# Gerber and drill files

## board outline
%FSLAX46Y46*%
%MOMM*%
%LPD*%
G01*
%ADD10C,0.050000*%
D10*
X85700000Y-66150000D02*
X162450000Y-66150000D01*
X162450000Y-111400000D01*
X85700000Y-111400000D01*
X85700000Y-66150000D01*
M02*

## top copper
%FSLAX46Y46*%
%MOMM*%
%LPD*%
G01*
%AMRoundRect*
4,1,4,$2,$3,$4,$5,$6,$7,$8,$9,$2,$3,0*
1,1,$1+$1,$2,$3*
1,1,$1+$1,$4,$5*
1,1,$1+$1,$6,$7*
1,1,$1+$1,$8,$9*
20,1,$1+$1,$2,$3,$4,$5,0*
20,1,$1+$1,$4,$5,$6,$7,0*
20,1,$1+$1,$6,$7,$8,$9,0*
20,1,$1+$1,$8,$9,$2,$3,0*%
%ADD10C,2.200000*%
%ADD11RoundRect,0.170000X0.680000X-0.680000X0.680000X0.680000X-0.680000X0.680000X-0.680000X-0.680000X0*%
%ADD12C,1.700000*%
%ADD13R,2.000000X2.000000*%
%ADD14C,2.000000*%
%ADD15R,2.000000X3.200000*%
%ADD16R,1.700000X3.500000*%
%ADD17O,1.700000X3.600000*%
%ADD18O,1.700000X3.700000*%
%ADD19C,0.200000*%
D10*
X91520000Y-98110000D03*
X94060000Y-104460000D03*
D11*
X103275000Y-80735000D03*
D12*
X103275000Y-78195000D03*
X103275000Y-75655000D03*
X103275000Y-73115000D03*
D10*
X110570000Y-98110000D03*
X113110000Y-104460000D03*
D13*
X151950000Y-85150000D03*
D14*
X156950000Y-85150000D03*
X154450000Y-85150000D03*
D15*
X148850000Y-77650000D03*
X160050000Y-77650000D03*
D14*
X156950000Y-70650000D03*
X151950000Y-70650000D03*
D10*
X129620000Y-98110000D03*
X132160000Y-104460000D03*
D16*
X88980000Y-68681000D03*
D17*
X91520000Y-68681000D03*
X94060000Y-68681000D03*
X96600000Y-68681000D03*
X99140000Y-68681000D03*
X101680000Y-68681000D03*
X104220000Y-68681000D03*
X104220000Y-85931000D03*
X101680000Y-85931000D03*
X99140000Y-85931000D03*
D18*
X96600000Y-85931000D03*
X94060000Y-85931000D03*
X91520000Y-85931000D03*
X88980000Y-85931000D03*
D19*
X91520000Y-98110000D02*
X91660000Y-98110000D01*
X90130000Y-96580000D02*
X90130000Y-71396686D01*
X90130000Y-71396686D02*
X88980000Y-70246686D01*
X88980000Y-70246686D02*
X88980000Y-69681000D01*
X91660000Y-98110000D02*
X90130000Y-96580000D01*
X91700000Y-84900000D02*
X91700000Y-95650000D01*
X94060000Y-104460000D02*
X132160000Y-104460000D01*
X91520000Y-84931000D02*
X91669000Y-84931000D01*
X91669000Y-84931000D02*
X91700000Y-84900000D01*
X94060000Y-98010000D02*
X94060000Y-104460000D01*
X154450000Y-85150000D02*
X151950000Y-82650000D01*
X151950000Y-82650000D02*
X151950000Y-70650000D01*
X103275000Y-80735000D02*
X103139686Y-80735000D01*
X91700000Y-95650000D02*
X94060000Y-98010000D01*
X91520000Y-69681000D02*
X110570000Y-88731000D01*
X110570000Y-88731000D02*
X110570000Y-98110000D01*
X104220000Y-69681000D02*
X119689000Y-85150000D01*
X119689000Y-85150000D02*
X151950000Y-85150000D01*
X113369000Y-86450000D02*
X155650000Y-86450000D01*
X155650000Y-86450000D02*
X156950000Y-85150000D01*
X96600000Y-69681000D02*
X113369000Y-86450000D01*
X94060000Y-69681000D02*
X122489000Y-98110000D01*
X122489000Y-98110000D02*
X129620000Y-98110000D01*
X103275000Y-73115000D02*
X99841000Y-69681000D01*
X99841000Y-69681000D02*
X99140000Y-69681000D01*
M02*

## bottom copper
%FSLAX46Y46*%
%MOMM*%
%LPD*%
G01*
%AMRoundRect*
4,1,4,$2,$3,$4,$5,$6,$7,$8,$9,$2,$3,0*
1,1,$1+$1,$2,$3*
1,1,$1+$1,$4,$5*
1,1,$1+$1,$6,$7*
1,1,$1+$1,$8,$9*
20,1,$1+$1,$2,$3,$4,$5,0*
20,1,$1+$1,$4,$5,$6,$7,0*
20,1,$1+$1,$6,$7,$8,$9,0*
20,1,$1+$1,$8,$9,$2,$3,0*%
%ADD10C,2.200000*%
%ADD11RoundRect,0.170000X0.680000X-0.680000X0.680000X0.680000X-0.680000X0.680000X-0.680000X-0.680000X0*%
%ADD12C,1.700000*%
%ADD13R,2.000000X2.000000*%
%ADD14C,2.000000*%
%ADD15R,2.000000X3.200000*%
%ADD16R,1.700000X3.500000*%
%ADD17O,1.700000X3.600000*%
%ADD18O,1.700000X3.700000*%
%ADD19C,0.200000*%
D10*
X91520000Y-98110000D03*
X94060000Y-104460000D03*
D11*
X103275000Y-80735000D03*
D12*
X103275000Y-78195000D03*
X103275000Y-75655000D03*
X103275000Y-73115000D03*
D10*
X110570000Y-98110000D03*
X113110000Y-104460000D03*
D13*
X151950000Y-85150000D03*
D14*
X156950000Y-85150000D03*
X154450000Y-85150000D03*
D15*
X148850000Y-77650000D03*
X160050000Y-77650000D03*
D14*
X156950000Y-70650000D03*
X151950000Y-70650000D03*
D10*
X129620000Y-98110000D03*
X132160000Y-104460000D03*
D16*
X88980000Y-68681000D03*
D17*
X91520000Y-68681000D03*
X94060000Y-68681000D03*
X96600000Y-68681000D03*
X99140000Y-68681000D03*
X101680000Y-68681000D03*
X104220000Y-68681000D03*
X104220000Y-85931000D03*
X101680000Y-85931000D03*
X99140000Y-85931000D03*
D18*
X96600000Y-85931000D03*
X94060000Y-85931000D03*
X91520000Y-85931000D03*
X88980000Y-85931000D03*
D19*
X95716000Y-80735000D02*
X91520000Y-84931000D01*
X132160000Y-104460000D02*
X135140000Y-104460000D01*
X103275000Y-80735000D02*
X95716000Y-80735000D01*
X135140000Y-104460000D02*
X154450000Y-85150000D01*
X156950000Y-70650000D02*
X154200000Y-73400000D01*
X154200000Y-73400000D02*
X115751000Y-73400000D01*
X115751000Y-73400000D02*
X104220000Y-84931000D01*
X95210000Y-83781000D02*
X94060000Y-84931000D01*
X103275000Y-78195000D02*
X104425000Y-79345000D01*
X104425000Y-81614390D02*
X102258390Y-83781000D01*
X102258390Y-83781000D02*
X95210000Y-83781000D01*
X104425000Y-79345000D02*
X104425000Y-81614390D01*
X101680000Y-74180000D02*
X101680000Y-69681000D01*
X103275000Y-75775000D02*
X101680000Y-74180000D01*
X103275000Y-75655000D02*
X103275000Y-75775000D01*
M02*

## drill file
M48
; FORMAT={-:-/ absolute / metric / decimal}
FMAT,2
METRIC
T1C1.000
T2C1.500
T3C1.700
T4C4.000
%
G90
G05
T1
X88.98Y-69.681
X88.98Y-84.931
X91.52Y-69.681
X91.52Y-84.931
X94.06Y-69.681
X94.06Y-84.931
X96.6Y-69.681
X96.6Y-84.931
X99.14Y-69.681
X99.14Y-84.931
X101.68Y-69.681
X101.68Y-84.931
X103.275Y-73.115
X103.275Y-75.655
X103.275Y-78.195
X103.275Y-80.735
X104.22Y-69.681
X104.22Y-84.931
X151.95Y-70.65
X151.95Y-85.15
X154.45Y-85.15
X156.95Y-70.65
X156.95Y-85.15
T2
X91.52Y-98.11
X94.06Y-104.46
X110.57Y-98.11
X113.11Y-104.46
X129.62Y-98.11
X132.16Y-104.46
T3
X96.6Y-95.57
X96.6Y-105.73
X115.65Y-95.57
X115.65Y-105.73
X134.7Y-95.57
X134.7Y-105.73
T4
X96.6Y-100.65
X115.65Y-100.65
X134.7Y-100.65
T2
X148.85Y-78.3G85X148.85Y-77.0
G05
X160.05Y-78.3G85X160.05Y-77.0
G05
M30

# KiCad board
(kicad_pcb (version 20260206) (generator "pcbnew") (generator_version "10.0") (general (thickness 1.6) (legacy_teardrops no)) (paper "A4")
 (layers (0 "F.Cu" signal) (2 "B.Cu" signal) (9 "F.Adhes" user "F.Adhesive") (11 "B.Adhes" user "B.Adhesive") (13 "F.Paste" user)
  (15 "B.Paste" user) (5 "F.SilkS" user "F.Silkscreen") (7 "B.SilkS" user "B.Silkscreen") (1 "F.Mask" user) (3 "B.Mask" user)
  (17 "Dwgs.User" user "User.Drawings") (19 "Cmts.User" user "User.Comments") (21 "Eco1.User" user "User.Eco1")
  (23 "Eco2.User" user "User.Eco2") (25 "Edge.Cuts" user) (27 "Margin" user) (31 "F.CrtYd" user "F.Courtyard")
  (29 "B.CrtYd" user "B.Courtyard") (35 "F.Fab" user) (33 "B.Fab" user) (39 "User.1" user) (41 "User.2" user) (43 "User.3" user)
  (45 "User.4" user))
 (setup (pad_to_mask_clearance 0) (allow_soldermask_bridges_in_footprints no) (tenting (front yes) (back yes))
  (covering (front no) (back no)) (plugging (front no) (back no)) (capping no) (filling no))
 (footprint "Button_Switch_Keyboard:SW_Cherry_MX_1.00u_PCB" (layer "F.Cu") (at 91.52 98.11 90)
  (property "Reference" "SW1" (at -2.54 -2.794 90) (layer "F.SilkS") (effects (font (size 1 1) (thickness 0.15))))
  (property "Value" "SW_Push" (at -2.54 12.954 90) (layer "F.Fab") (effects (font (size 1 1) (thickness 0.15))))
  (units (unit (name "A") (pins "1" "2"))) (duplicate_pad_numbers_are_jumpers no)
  (pad "" np_thru_hole circle (at -7.62 5.08 90) (size 1.7 1.7) (drill 1.7) (layers "*.Cu" "*.Mask"))
  (pad "" np_thru_hole circle (at -2.54 5.08 90) (size 4 4) (drill 4) (layers "*.Cu" "*.Mask"))
  (pad "" np_thru_hole circle (at 2.54 5.08 90) (size 1.7 1.7) (drill 1.7) (layers "*.Cu" "*.Mask"))
  (pad "1" thru_hole circle (at 0 0 90) (size 2.2 2.2) (drill 1.5) (layers "*.Cu" "*.Mask") (remove_unused_layers no)
   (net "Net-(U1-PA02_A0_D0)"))
  (pad "2" thru_hole circle (at -6.35 2.54 90) (size 2.2 2.2) (drill 1.5) (layers "*.Cu" "*.Mask") (remove_unused_layers no) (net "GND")))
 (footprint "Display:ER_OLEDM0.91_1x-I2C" (layer "F.Cu") (at 103.275 80.735 90)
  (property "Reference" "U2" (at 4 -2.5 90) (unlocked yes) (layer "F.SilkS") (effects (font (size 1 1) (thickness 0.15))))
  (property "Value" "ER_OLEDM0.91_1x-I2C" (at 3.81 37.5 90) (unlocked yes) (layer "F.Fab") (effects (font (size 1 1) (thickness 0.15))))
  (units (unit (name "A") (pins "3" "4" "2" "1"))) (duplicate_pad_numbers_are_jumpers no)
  (pad "1" thru_hole roundrect (at 0 0 90) (size 1.7 1.7) (drill 1) (layers "*.Cu" "*.Mask") (remove_unused_layers no)
   (roundrect_rratio 0.1) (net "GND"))
  (pad "2" thru_hole circle (at 2.54 0 90) (size 1.7 1.7) (drill 1) (layers "*.Cu" "*.Mask") (remove_unused_layers no) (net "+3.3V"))
  (pad "3" thru_hole circle (at 5.08 0 90) (size 1.7 1.7) (drill 1) (layers "*.Cu" "*.Mask") (remove_unused_layers no)
   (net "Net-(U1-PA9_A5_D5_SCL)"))
  (pad "4" thru_hole circle (at 7.62 0 90) (size 1.7 1.7) (drill 1) (layers "*.Cu" "*.Mask") (remove_unused_layers no)
   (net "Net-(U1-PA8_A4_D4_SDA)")))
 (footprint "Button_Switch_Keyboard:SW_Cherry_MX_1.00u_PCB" (layer "F.Cu") (at 110.57 98.11 90)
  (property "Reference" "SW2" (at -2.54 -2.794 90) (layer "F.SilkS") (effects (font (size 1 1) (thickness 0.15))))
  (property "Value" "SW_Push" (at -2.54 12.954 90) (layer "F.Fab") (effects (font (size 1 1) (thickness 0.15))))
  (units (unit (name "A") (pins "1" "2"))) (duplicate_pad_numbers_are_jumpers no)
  (pad "" np_thru_hole circle (at -7.62 5.08 90) (size 1.7 1.7) (drill 1.7) (layers "*.Cu" "*.Mask"))
  (pad "" np_thru_hole circle (at -2.54 5.08 90) (size 4 4) (drill 4) (layers "*.Cu" "*.Mask"))
  (pad "" np_thru_hole circle (at 2.54 5.08 90) (size 1.7 1.7) (drill 1.7) (layers "*.Cu" "*.Mask"))
  (pad "1" thru_hole circle (at 0 0 90) (size 2.2 2.2) (drill 1.5) (layers "*.Cu" "*.Mask") (remove_unused_layers no)
   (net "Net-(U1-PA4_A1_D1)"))
  (pad "2" thru_hole circle (at -6.35 2.54 90) (size 2.2 2.2) (drill 1.5) (layers "*.Cu" "*.Mask") (remove_unused_layers no) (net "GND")))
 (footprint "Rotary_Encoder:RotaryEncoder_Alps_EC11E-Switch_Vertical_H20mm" (layer "F.Cu") (at 151.95 85.15 90)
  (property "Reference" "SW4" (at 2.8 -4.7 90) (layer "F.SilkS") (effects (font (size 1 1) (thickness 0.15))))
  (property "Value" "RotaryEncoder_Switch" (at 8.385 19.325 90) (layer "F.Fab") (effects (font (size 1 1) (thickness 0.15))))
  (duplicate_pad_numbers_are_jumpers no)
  (pad "A" thru_hole rect (at 0 0 90) (size 2 2) (drill 1) (layers "*.Cu" "*.Mask") (remove_unused_layers no) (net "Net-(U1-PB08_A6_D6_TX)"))
  (pad "B" thru_hole circle (at 0 5 90) (size 2 2) (drill 1) (layers "*.Cu" "*.Mask") (remove_unused_layers no) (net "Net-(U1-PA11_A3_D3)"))
  (pad "C" thru_hole circle (at 0 2.5 90) (size 2 2) (drill 1) (layers "*.Cu" "*.Mask") (remove_unused_layers no) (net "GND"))
  (pad "MP" thru_hole rect (at 7.5 -3.1 90) (size 3.2 2) (drill oval 2.8 1.5) (layers "*.Cu" "*.Mask") (remove_unused_layers no))
  (pad "MP" thru_hole rect (at 7.5 8.1 90) (size 3.2 2) (drill oval 2.8 1.5) (layers "*.Cu" "*.Mask") (remove_unused_layers no))
  (pad "S1" thru_hole circle (at 14.5 5 90) (size 2 2) (drill 1) (layers "*.Cu" "*.Mask") (remove_unused_layers no)
   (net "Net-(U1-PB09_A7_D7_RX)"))
  (pad "S2" thru_hole circle (at 14.5 0 90) (size 2 2) (drill 1) (layers "*.Cu" "*.Mask") (remove_unused_layers no) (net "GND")))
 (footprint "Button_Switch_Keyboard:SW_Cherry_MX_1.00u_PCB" (layer "F.Cu") (at 129.62 98.11 90)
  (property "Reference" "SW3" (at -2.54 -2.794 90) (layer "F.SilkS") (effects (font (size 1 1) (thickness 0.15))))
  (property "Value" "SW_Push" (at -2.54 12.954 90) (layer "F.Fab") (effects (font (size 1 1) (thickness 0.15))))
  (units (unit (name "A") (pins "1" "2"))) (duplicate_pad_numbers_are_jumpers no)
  (pad "" np_thru_hole circle (at -7.62 5.08 90) (size 1.7 1.7) (drill 1.7) (layers "*.Cu" "*.Mask"))
  (pad "" np_thru_hole circle (at -2.54 5.08 90) (size 4 4) (drill 4) (layers "*.Cu" "*.Mask"))
  (pad "" np_thru_hole circle (at 2.54 5.08 90) (size 1.7 1.7) (drill 1.7) (layers "*.Cu" "*.Mask"))
  (pad "1" thru_hole circle (at 0 0 90) (size 2.2 2.2) (drill 1.5) (layers "*.Cu" "*.Mask") (remove_unused_layers no)
   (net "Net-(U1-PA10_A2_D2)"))
  (pad "2" thru_hole circle (at -6.35 2.54 90) (size 2.2 2.2) (drill 1.5) (layers "*.Cu" "*.Mask") (remove_unused_layers no) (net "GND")))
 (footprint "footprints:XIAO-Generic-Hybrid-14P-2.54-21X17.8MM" (layer "B.Cu") (at 96.6 77.306 -90)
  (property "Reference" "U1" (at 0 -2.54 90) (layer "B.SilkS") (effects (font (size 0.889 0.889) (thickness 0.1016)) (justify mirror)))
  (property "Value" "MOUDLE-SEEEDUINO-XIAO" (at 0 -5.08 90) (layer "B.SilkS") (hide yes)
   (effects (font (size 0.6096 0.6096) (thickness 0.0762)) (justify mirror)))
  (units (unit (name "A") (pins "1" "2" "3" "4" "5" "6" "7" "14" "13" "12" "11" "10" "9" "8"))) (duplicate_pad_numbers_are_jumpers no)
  (pad "1" thru_hole rect (at -7.625 7.62 270) (size 3.5 1.7) (drill 1 (offset -1 0)) (layers "*.Cu" "*.Mask") (remove_unused_layers no)
   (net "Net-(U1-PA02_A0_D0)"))
  (pad "2" thru_hole oval (at -7.625 5.08 270) (size 3.6 1.7) (drill 1 (offset -1 0)) (layers "*.Cu" "*.Mask") (remove_unused_layers no)
   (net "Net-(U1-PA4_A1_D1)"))
  (pad "3" thru_hole oval (at -7.625 2.54 270) (size 3.6 1.7) (drill 1 (offset -1 0)) (layers "*.Cu" "*.Mask") (remove_unused_layers no)
   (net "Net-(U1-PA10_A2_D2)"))
  (pad "4" thru_hole oval (at -7.625 0 270) (size 3.6 1.7) (drill 1 (offset -1 0)) (layers "*.Cu" "*.Mask") (remove_unused_layers no)
   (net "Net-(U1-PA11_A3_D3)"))
  (pad "5" thru_hole oval (at -7.625 -2.54 270) (size 3.6 1.7) (drill 1 (offset -1 0)) (layers "*.Cu" "*.Mask") (remove_unused_layers no)
   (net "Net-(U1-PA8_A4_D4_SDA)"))
  (pad "6" thru_hole oval (at -7.625 -5.08 90) (size 3.6 1.7) (drill 1 (offset 1 0)) (layers "*.Cu" "*.Mask") (remove_unused_layers no)
   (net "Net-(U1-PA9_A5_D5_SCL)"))
  (pad "7" thru_hole oval (at -7.625 -7.62 270) (size 3.6 1.7) (drill 1 (offset -1 0)) (layers "*.Cu" "*.Mask") (remove_unused_layers no)
   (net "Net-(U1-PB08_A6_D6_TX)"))
  (pad "8" thru_hole oval (at 7.625 -7.62 270) (size 3.6 1.7) (drill 1 (offset 1 0)) (layers "*.Cu" "*.Mask") (remove_unused_layers no)
   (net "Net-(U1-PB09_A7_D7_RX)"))
  (pad "9" thru_hole oval (at 7.625 -5.08 270) (size 3.6 1.7) (drill 1 (offset 1 0)) (layers "*.Cu" "*.Mask") (remove_unused_layers no)
   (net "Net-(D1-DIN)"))
  (pad "10" thru_hole oval (at 7.625 -2.54 270) (size 3.6 1.7) (drill 1 (offset 1 0)) (layers "*.Cu" "*.Mask") (remove_unused_layers no)
   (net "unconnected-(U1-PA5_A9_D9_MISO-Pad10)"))
  (pad "11" thru_hole oval (at 7.625 0 270) (size 3.7 1.7) (drill 1 (offset 1 0)) (layers "*.Cu" "*.Mask") (remove_unused_layers no)
   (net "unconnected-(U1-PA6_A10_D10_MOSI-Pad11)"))
  (pad "12" thru_hole oval (at 7.625 2.54 270) (size 3.7 1.7) (drill 1 (offset 1 0)) (layers "*.Cu" "*.Mask") (remove_unused_layers no)
   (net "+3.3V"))
  (pad "13" thru_hole oval (at 7.625 5.08 270) (size 3.7 1.7) (drill 1 (offset 1 0)) (layers "*.Cu" "*.Mask") (remove_unused_layers no)
   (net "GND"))
  (pad "14" thru_hole oval (at 7.625 7.62 270) (size 3.7 1.7) (drill 1 (offset 1 0)) (layers "*.Cu" "*.Mask") (remove_unused_layers no)
   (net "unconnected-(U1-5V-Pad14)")))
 (gr_rect (start 85.7 66.15) (end 162.45 111.4) (stroke (width 0.05) (type default)) (fill no) (layer "Edge.Cuts"))
 (segment (start 91.52 98.11) (end 91.66 98.11) (width 0.2) (layer "F.Cu") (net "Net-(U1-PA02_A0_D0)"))
 (segment (start 90.13 96.58) (end 90.13 71.396686) (width 0.2) (layer "F.Cu") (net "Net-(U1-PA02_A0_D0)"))
 (segment (start 90.13 71.396686) (end 88.98 70.246686) (width 0.2) (layer "F.Cu") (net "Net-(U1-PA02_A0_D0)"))
 (segment (start 88.98 70.246686) (end 88.98 69.681) (width 0.2) (layer "F.Cu") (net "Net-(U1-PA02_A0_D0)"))
 (segment (start 91.66 98.11) (end 90.13 96.58) (width 0.2) (layer "F.Cu") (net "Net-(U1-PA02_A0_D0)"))
 (segment (start 91.7 84.9) (end 91.7 95.65) (width 0.2) (layer "F.Cu") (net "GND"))
 (segment (start 94.06 104.46) (end 132.16 104.46) (width 0.2) (layer "F.Cu") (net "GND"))
 (segment (start 91.52 84.931) (end 91.669 84.931) (width 0.2) (layer "F.Cu") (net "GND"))
 (segment (start 91.669 84.931) (end 91.7 84.9) (width 0.2) (layer "F.Cu") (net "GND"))
 (segment (start 94.06 98.01) (end 94.06 104.46) (width 0.2) (layer "F.Cu") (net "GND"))
 (segment (start 154.45 85.15) (end 151.95 82.65) (width 0.2) (layer "F.Cu") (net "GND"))
 (segment (start 151.95 82.65) (end 151.95 70.65) (width 0.2) (layer "F.Cu") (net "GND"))
 (segment (start 103.275 80.735) (end 103.139686 80.735) (width 0.2) (layer "F.Cu") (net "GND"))
 (segment (start 91.7 95.65) (end 94.06 98.01) (width 0.2) (layer "F.Cu") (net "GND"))
 (segment (start 95.716 80.735) (end 91.52 84.931) (width 0.2) (layer "B.Cu") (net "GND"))
 (segment (start 132.16 104.46) (end 135.14 104.46) (width 0.2) (layer "B.Cu") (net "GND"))
 (segment (start 103.275 80.735) (end 95.716 80.735) (width 0.2) (layer "B.Cu") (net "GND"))
 (segment (start 135.14 104.46) (end 154.45 85.15) (width 0.2) (layer "B.Cu") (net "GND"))
 (segment (start 91.52 69.681) (end 110.57 88.731) (width 0.2) (layer "F.Cu") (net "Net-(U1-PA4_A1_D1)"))
 (segment (start 110.57 88.731) (end 110.57 98.11) (width 0.2) (layer "F.Cu") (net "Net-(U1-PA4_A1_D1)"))
 (segment (start 104.22 69.681) (end 119.689 85.15) (width 0.2) (layer "F.Cu") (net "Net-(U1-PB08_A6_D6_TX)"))
 (segment (start 119.689 85.15) (end 151.95 85.15) (width 0.2) (layer "F.Cu") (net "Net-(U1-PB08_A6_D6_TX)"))
 (segment (start 113.369 86.45) (end 155.65 86.45) (width 0.2) (layer "F.Cu") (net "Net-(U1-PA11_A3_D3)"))
 (segment (start 155.65 86.45) (end 156.95 85.15) (width 0.2) (layer "F.Cu") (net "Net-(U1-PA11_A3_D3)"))
 (segment (start 96.6 69.681) (end 113.369 86.45) (width 0.2) (layer "F.Cu") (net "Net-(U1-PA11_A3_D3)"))
 (segment (start 156.95 70.65) (end 154.2 73.4) (width 0.2) (layer "B.Cu") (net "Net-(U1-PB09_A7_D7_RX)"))
 (segment (start 154.2 73.4) (end 115.751 73.4) (width 0.2) (layer "B.Cu") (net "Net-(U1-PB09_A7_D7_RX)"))
 (segment (start 115.751 73.4) (end 104.22 84.931) (width 0.2) (layer "B.Cu") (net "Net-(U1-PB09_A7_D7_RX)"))
 (segment (start 94.06 69.681) (end 122.489 98.11) (width 0.2) (layer "F.Cu") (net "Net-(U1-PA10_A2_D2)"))
 (segment (start 122.489 98.11) (end 129.62 98.11) (width 0.2) (layer "F.Cu") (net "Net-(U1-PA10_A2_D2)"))
 (segment (start 103.275 73.115) (end 99.841 69.681) (width 0.2) (layer "F.Cu") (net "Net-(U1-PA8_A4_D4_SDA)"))
 (segment (start 99.841 69.681) (end 99.14 69.681) (width 0.2) (layer "F.Cu") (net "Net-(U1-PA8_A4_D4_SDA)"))
 (segment (start 95.21 83.781) (end 94.06 84.931) (width 0.2) (layer "B.Cu") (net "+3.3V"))
 (segment (start 103.275 78.195) (end 104.425 79.345) (width 0.2) (layer "B.Cu") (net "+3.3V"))
 (segment (start 104.425 81.61439) (end 102.25839 83.781) (width 0.2) (layer "B.Cu") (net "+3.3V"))
 (segment (start 102.25839 83.781) (end 95.21 83.781) (width 0.2) (layer "B.Cu") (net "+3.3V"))
 (segment (start 104.425 79.345) (end 104.425 81.61439) (width 0.2) (layer "B.Cu") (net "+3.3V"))
 (segment (start 101.68 74.18) (end 101.68 69.681) (width 0.2) (layer "B.Cu") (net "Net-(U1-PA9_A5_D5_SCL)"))
 (segment (start 103.275 75.775) (end 101.68 74.18) (width 0.2) (layer "B.Cu") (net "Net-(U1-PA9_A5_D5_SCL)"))
 (segment (start 103.275 75.655) (end 103.275 75.775) (width 0.2) (layer "B.Cu") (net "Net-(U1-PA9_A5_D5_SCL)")))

